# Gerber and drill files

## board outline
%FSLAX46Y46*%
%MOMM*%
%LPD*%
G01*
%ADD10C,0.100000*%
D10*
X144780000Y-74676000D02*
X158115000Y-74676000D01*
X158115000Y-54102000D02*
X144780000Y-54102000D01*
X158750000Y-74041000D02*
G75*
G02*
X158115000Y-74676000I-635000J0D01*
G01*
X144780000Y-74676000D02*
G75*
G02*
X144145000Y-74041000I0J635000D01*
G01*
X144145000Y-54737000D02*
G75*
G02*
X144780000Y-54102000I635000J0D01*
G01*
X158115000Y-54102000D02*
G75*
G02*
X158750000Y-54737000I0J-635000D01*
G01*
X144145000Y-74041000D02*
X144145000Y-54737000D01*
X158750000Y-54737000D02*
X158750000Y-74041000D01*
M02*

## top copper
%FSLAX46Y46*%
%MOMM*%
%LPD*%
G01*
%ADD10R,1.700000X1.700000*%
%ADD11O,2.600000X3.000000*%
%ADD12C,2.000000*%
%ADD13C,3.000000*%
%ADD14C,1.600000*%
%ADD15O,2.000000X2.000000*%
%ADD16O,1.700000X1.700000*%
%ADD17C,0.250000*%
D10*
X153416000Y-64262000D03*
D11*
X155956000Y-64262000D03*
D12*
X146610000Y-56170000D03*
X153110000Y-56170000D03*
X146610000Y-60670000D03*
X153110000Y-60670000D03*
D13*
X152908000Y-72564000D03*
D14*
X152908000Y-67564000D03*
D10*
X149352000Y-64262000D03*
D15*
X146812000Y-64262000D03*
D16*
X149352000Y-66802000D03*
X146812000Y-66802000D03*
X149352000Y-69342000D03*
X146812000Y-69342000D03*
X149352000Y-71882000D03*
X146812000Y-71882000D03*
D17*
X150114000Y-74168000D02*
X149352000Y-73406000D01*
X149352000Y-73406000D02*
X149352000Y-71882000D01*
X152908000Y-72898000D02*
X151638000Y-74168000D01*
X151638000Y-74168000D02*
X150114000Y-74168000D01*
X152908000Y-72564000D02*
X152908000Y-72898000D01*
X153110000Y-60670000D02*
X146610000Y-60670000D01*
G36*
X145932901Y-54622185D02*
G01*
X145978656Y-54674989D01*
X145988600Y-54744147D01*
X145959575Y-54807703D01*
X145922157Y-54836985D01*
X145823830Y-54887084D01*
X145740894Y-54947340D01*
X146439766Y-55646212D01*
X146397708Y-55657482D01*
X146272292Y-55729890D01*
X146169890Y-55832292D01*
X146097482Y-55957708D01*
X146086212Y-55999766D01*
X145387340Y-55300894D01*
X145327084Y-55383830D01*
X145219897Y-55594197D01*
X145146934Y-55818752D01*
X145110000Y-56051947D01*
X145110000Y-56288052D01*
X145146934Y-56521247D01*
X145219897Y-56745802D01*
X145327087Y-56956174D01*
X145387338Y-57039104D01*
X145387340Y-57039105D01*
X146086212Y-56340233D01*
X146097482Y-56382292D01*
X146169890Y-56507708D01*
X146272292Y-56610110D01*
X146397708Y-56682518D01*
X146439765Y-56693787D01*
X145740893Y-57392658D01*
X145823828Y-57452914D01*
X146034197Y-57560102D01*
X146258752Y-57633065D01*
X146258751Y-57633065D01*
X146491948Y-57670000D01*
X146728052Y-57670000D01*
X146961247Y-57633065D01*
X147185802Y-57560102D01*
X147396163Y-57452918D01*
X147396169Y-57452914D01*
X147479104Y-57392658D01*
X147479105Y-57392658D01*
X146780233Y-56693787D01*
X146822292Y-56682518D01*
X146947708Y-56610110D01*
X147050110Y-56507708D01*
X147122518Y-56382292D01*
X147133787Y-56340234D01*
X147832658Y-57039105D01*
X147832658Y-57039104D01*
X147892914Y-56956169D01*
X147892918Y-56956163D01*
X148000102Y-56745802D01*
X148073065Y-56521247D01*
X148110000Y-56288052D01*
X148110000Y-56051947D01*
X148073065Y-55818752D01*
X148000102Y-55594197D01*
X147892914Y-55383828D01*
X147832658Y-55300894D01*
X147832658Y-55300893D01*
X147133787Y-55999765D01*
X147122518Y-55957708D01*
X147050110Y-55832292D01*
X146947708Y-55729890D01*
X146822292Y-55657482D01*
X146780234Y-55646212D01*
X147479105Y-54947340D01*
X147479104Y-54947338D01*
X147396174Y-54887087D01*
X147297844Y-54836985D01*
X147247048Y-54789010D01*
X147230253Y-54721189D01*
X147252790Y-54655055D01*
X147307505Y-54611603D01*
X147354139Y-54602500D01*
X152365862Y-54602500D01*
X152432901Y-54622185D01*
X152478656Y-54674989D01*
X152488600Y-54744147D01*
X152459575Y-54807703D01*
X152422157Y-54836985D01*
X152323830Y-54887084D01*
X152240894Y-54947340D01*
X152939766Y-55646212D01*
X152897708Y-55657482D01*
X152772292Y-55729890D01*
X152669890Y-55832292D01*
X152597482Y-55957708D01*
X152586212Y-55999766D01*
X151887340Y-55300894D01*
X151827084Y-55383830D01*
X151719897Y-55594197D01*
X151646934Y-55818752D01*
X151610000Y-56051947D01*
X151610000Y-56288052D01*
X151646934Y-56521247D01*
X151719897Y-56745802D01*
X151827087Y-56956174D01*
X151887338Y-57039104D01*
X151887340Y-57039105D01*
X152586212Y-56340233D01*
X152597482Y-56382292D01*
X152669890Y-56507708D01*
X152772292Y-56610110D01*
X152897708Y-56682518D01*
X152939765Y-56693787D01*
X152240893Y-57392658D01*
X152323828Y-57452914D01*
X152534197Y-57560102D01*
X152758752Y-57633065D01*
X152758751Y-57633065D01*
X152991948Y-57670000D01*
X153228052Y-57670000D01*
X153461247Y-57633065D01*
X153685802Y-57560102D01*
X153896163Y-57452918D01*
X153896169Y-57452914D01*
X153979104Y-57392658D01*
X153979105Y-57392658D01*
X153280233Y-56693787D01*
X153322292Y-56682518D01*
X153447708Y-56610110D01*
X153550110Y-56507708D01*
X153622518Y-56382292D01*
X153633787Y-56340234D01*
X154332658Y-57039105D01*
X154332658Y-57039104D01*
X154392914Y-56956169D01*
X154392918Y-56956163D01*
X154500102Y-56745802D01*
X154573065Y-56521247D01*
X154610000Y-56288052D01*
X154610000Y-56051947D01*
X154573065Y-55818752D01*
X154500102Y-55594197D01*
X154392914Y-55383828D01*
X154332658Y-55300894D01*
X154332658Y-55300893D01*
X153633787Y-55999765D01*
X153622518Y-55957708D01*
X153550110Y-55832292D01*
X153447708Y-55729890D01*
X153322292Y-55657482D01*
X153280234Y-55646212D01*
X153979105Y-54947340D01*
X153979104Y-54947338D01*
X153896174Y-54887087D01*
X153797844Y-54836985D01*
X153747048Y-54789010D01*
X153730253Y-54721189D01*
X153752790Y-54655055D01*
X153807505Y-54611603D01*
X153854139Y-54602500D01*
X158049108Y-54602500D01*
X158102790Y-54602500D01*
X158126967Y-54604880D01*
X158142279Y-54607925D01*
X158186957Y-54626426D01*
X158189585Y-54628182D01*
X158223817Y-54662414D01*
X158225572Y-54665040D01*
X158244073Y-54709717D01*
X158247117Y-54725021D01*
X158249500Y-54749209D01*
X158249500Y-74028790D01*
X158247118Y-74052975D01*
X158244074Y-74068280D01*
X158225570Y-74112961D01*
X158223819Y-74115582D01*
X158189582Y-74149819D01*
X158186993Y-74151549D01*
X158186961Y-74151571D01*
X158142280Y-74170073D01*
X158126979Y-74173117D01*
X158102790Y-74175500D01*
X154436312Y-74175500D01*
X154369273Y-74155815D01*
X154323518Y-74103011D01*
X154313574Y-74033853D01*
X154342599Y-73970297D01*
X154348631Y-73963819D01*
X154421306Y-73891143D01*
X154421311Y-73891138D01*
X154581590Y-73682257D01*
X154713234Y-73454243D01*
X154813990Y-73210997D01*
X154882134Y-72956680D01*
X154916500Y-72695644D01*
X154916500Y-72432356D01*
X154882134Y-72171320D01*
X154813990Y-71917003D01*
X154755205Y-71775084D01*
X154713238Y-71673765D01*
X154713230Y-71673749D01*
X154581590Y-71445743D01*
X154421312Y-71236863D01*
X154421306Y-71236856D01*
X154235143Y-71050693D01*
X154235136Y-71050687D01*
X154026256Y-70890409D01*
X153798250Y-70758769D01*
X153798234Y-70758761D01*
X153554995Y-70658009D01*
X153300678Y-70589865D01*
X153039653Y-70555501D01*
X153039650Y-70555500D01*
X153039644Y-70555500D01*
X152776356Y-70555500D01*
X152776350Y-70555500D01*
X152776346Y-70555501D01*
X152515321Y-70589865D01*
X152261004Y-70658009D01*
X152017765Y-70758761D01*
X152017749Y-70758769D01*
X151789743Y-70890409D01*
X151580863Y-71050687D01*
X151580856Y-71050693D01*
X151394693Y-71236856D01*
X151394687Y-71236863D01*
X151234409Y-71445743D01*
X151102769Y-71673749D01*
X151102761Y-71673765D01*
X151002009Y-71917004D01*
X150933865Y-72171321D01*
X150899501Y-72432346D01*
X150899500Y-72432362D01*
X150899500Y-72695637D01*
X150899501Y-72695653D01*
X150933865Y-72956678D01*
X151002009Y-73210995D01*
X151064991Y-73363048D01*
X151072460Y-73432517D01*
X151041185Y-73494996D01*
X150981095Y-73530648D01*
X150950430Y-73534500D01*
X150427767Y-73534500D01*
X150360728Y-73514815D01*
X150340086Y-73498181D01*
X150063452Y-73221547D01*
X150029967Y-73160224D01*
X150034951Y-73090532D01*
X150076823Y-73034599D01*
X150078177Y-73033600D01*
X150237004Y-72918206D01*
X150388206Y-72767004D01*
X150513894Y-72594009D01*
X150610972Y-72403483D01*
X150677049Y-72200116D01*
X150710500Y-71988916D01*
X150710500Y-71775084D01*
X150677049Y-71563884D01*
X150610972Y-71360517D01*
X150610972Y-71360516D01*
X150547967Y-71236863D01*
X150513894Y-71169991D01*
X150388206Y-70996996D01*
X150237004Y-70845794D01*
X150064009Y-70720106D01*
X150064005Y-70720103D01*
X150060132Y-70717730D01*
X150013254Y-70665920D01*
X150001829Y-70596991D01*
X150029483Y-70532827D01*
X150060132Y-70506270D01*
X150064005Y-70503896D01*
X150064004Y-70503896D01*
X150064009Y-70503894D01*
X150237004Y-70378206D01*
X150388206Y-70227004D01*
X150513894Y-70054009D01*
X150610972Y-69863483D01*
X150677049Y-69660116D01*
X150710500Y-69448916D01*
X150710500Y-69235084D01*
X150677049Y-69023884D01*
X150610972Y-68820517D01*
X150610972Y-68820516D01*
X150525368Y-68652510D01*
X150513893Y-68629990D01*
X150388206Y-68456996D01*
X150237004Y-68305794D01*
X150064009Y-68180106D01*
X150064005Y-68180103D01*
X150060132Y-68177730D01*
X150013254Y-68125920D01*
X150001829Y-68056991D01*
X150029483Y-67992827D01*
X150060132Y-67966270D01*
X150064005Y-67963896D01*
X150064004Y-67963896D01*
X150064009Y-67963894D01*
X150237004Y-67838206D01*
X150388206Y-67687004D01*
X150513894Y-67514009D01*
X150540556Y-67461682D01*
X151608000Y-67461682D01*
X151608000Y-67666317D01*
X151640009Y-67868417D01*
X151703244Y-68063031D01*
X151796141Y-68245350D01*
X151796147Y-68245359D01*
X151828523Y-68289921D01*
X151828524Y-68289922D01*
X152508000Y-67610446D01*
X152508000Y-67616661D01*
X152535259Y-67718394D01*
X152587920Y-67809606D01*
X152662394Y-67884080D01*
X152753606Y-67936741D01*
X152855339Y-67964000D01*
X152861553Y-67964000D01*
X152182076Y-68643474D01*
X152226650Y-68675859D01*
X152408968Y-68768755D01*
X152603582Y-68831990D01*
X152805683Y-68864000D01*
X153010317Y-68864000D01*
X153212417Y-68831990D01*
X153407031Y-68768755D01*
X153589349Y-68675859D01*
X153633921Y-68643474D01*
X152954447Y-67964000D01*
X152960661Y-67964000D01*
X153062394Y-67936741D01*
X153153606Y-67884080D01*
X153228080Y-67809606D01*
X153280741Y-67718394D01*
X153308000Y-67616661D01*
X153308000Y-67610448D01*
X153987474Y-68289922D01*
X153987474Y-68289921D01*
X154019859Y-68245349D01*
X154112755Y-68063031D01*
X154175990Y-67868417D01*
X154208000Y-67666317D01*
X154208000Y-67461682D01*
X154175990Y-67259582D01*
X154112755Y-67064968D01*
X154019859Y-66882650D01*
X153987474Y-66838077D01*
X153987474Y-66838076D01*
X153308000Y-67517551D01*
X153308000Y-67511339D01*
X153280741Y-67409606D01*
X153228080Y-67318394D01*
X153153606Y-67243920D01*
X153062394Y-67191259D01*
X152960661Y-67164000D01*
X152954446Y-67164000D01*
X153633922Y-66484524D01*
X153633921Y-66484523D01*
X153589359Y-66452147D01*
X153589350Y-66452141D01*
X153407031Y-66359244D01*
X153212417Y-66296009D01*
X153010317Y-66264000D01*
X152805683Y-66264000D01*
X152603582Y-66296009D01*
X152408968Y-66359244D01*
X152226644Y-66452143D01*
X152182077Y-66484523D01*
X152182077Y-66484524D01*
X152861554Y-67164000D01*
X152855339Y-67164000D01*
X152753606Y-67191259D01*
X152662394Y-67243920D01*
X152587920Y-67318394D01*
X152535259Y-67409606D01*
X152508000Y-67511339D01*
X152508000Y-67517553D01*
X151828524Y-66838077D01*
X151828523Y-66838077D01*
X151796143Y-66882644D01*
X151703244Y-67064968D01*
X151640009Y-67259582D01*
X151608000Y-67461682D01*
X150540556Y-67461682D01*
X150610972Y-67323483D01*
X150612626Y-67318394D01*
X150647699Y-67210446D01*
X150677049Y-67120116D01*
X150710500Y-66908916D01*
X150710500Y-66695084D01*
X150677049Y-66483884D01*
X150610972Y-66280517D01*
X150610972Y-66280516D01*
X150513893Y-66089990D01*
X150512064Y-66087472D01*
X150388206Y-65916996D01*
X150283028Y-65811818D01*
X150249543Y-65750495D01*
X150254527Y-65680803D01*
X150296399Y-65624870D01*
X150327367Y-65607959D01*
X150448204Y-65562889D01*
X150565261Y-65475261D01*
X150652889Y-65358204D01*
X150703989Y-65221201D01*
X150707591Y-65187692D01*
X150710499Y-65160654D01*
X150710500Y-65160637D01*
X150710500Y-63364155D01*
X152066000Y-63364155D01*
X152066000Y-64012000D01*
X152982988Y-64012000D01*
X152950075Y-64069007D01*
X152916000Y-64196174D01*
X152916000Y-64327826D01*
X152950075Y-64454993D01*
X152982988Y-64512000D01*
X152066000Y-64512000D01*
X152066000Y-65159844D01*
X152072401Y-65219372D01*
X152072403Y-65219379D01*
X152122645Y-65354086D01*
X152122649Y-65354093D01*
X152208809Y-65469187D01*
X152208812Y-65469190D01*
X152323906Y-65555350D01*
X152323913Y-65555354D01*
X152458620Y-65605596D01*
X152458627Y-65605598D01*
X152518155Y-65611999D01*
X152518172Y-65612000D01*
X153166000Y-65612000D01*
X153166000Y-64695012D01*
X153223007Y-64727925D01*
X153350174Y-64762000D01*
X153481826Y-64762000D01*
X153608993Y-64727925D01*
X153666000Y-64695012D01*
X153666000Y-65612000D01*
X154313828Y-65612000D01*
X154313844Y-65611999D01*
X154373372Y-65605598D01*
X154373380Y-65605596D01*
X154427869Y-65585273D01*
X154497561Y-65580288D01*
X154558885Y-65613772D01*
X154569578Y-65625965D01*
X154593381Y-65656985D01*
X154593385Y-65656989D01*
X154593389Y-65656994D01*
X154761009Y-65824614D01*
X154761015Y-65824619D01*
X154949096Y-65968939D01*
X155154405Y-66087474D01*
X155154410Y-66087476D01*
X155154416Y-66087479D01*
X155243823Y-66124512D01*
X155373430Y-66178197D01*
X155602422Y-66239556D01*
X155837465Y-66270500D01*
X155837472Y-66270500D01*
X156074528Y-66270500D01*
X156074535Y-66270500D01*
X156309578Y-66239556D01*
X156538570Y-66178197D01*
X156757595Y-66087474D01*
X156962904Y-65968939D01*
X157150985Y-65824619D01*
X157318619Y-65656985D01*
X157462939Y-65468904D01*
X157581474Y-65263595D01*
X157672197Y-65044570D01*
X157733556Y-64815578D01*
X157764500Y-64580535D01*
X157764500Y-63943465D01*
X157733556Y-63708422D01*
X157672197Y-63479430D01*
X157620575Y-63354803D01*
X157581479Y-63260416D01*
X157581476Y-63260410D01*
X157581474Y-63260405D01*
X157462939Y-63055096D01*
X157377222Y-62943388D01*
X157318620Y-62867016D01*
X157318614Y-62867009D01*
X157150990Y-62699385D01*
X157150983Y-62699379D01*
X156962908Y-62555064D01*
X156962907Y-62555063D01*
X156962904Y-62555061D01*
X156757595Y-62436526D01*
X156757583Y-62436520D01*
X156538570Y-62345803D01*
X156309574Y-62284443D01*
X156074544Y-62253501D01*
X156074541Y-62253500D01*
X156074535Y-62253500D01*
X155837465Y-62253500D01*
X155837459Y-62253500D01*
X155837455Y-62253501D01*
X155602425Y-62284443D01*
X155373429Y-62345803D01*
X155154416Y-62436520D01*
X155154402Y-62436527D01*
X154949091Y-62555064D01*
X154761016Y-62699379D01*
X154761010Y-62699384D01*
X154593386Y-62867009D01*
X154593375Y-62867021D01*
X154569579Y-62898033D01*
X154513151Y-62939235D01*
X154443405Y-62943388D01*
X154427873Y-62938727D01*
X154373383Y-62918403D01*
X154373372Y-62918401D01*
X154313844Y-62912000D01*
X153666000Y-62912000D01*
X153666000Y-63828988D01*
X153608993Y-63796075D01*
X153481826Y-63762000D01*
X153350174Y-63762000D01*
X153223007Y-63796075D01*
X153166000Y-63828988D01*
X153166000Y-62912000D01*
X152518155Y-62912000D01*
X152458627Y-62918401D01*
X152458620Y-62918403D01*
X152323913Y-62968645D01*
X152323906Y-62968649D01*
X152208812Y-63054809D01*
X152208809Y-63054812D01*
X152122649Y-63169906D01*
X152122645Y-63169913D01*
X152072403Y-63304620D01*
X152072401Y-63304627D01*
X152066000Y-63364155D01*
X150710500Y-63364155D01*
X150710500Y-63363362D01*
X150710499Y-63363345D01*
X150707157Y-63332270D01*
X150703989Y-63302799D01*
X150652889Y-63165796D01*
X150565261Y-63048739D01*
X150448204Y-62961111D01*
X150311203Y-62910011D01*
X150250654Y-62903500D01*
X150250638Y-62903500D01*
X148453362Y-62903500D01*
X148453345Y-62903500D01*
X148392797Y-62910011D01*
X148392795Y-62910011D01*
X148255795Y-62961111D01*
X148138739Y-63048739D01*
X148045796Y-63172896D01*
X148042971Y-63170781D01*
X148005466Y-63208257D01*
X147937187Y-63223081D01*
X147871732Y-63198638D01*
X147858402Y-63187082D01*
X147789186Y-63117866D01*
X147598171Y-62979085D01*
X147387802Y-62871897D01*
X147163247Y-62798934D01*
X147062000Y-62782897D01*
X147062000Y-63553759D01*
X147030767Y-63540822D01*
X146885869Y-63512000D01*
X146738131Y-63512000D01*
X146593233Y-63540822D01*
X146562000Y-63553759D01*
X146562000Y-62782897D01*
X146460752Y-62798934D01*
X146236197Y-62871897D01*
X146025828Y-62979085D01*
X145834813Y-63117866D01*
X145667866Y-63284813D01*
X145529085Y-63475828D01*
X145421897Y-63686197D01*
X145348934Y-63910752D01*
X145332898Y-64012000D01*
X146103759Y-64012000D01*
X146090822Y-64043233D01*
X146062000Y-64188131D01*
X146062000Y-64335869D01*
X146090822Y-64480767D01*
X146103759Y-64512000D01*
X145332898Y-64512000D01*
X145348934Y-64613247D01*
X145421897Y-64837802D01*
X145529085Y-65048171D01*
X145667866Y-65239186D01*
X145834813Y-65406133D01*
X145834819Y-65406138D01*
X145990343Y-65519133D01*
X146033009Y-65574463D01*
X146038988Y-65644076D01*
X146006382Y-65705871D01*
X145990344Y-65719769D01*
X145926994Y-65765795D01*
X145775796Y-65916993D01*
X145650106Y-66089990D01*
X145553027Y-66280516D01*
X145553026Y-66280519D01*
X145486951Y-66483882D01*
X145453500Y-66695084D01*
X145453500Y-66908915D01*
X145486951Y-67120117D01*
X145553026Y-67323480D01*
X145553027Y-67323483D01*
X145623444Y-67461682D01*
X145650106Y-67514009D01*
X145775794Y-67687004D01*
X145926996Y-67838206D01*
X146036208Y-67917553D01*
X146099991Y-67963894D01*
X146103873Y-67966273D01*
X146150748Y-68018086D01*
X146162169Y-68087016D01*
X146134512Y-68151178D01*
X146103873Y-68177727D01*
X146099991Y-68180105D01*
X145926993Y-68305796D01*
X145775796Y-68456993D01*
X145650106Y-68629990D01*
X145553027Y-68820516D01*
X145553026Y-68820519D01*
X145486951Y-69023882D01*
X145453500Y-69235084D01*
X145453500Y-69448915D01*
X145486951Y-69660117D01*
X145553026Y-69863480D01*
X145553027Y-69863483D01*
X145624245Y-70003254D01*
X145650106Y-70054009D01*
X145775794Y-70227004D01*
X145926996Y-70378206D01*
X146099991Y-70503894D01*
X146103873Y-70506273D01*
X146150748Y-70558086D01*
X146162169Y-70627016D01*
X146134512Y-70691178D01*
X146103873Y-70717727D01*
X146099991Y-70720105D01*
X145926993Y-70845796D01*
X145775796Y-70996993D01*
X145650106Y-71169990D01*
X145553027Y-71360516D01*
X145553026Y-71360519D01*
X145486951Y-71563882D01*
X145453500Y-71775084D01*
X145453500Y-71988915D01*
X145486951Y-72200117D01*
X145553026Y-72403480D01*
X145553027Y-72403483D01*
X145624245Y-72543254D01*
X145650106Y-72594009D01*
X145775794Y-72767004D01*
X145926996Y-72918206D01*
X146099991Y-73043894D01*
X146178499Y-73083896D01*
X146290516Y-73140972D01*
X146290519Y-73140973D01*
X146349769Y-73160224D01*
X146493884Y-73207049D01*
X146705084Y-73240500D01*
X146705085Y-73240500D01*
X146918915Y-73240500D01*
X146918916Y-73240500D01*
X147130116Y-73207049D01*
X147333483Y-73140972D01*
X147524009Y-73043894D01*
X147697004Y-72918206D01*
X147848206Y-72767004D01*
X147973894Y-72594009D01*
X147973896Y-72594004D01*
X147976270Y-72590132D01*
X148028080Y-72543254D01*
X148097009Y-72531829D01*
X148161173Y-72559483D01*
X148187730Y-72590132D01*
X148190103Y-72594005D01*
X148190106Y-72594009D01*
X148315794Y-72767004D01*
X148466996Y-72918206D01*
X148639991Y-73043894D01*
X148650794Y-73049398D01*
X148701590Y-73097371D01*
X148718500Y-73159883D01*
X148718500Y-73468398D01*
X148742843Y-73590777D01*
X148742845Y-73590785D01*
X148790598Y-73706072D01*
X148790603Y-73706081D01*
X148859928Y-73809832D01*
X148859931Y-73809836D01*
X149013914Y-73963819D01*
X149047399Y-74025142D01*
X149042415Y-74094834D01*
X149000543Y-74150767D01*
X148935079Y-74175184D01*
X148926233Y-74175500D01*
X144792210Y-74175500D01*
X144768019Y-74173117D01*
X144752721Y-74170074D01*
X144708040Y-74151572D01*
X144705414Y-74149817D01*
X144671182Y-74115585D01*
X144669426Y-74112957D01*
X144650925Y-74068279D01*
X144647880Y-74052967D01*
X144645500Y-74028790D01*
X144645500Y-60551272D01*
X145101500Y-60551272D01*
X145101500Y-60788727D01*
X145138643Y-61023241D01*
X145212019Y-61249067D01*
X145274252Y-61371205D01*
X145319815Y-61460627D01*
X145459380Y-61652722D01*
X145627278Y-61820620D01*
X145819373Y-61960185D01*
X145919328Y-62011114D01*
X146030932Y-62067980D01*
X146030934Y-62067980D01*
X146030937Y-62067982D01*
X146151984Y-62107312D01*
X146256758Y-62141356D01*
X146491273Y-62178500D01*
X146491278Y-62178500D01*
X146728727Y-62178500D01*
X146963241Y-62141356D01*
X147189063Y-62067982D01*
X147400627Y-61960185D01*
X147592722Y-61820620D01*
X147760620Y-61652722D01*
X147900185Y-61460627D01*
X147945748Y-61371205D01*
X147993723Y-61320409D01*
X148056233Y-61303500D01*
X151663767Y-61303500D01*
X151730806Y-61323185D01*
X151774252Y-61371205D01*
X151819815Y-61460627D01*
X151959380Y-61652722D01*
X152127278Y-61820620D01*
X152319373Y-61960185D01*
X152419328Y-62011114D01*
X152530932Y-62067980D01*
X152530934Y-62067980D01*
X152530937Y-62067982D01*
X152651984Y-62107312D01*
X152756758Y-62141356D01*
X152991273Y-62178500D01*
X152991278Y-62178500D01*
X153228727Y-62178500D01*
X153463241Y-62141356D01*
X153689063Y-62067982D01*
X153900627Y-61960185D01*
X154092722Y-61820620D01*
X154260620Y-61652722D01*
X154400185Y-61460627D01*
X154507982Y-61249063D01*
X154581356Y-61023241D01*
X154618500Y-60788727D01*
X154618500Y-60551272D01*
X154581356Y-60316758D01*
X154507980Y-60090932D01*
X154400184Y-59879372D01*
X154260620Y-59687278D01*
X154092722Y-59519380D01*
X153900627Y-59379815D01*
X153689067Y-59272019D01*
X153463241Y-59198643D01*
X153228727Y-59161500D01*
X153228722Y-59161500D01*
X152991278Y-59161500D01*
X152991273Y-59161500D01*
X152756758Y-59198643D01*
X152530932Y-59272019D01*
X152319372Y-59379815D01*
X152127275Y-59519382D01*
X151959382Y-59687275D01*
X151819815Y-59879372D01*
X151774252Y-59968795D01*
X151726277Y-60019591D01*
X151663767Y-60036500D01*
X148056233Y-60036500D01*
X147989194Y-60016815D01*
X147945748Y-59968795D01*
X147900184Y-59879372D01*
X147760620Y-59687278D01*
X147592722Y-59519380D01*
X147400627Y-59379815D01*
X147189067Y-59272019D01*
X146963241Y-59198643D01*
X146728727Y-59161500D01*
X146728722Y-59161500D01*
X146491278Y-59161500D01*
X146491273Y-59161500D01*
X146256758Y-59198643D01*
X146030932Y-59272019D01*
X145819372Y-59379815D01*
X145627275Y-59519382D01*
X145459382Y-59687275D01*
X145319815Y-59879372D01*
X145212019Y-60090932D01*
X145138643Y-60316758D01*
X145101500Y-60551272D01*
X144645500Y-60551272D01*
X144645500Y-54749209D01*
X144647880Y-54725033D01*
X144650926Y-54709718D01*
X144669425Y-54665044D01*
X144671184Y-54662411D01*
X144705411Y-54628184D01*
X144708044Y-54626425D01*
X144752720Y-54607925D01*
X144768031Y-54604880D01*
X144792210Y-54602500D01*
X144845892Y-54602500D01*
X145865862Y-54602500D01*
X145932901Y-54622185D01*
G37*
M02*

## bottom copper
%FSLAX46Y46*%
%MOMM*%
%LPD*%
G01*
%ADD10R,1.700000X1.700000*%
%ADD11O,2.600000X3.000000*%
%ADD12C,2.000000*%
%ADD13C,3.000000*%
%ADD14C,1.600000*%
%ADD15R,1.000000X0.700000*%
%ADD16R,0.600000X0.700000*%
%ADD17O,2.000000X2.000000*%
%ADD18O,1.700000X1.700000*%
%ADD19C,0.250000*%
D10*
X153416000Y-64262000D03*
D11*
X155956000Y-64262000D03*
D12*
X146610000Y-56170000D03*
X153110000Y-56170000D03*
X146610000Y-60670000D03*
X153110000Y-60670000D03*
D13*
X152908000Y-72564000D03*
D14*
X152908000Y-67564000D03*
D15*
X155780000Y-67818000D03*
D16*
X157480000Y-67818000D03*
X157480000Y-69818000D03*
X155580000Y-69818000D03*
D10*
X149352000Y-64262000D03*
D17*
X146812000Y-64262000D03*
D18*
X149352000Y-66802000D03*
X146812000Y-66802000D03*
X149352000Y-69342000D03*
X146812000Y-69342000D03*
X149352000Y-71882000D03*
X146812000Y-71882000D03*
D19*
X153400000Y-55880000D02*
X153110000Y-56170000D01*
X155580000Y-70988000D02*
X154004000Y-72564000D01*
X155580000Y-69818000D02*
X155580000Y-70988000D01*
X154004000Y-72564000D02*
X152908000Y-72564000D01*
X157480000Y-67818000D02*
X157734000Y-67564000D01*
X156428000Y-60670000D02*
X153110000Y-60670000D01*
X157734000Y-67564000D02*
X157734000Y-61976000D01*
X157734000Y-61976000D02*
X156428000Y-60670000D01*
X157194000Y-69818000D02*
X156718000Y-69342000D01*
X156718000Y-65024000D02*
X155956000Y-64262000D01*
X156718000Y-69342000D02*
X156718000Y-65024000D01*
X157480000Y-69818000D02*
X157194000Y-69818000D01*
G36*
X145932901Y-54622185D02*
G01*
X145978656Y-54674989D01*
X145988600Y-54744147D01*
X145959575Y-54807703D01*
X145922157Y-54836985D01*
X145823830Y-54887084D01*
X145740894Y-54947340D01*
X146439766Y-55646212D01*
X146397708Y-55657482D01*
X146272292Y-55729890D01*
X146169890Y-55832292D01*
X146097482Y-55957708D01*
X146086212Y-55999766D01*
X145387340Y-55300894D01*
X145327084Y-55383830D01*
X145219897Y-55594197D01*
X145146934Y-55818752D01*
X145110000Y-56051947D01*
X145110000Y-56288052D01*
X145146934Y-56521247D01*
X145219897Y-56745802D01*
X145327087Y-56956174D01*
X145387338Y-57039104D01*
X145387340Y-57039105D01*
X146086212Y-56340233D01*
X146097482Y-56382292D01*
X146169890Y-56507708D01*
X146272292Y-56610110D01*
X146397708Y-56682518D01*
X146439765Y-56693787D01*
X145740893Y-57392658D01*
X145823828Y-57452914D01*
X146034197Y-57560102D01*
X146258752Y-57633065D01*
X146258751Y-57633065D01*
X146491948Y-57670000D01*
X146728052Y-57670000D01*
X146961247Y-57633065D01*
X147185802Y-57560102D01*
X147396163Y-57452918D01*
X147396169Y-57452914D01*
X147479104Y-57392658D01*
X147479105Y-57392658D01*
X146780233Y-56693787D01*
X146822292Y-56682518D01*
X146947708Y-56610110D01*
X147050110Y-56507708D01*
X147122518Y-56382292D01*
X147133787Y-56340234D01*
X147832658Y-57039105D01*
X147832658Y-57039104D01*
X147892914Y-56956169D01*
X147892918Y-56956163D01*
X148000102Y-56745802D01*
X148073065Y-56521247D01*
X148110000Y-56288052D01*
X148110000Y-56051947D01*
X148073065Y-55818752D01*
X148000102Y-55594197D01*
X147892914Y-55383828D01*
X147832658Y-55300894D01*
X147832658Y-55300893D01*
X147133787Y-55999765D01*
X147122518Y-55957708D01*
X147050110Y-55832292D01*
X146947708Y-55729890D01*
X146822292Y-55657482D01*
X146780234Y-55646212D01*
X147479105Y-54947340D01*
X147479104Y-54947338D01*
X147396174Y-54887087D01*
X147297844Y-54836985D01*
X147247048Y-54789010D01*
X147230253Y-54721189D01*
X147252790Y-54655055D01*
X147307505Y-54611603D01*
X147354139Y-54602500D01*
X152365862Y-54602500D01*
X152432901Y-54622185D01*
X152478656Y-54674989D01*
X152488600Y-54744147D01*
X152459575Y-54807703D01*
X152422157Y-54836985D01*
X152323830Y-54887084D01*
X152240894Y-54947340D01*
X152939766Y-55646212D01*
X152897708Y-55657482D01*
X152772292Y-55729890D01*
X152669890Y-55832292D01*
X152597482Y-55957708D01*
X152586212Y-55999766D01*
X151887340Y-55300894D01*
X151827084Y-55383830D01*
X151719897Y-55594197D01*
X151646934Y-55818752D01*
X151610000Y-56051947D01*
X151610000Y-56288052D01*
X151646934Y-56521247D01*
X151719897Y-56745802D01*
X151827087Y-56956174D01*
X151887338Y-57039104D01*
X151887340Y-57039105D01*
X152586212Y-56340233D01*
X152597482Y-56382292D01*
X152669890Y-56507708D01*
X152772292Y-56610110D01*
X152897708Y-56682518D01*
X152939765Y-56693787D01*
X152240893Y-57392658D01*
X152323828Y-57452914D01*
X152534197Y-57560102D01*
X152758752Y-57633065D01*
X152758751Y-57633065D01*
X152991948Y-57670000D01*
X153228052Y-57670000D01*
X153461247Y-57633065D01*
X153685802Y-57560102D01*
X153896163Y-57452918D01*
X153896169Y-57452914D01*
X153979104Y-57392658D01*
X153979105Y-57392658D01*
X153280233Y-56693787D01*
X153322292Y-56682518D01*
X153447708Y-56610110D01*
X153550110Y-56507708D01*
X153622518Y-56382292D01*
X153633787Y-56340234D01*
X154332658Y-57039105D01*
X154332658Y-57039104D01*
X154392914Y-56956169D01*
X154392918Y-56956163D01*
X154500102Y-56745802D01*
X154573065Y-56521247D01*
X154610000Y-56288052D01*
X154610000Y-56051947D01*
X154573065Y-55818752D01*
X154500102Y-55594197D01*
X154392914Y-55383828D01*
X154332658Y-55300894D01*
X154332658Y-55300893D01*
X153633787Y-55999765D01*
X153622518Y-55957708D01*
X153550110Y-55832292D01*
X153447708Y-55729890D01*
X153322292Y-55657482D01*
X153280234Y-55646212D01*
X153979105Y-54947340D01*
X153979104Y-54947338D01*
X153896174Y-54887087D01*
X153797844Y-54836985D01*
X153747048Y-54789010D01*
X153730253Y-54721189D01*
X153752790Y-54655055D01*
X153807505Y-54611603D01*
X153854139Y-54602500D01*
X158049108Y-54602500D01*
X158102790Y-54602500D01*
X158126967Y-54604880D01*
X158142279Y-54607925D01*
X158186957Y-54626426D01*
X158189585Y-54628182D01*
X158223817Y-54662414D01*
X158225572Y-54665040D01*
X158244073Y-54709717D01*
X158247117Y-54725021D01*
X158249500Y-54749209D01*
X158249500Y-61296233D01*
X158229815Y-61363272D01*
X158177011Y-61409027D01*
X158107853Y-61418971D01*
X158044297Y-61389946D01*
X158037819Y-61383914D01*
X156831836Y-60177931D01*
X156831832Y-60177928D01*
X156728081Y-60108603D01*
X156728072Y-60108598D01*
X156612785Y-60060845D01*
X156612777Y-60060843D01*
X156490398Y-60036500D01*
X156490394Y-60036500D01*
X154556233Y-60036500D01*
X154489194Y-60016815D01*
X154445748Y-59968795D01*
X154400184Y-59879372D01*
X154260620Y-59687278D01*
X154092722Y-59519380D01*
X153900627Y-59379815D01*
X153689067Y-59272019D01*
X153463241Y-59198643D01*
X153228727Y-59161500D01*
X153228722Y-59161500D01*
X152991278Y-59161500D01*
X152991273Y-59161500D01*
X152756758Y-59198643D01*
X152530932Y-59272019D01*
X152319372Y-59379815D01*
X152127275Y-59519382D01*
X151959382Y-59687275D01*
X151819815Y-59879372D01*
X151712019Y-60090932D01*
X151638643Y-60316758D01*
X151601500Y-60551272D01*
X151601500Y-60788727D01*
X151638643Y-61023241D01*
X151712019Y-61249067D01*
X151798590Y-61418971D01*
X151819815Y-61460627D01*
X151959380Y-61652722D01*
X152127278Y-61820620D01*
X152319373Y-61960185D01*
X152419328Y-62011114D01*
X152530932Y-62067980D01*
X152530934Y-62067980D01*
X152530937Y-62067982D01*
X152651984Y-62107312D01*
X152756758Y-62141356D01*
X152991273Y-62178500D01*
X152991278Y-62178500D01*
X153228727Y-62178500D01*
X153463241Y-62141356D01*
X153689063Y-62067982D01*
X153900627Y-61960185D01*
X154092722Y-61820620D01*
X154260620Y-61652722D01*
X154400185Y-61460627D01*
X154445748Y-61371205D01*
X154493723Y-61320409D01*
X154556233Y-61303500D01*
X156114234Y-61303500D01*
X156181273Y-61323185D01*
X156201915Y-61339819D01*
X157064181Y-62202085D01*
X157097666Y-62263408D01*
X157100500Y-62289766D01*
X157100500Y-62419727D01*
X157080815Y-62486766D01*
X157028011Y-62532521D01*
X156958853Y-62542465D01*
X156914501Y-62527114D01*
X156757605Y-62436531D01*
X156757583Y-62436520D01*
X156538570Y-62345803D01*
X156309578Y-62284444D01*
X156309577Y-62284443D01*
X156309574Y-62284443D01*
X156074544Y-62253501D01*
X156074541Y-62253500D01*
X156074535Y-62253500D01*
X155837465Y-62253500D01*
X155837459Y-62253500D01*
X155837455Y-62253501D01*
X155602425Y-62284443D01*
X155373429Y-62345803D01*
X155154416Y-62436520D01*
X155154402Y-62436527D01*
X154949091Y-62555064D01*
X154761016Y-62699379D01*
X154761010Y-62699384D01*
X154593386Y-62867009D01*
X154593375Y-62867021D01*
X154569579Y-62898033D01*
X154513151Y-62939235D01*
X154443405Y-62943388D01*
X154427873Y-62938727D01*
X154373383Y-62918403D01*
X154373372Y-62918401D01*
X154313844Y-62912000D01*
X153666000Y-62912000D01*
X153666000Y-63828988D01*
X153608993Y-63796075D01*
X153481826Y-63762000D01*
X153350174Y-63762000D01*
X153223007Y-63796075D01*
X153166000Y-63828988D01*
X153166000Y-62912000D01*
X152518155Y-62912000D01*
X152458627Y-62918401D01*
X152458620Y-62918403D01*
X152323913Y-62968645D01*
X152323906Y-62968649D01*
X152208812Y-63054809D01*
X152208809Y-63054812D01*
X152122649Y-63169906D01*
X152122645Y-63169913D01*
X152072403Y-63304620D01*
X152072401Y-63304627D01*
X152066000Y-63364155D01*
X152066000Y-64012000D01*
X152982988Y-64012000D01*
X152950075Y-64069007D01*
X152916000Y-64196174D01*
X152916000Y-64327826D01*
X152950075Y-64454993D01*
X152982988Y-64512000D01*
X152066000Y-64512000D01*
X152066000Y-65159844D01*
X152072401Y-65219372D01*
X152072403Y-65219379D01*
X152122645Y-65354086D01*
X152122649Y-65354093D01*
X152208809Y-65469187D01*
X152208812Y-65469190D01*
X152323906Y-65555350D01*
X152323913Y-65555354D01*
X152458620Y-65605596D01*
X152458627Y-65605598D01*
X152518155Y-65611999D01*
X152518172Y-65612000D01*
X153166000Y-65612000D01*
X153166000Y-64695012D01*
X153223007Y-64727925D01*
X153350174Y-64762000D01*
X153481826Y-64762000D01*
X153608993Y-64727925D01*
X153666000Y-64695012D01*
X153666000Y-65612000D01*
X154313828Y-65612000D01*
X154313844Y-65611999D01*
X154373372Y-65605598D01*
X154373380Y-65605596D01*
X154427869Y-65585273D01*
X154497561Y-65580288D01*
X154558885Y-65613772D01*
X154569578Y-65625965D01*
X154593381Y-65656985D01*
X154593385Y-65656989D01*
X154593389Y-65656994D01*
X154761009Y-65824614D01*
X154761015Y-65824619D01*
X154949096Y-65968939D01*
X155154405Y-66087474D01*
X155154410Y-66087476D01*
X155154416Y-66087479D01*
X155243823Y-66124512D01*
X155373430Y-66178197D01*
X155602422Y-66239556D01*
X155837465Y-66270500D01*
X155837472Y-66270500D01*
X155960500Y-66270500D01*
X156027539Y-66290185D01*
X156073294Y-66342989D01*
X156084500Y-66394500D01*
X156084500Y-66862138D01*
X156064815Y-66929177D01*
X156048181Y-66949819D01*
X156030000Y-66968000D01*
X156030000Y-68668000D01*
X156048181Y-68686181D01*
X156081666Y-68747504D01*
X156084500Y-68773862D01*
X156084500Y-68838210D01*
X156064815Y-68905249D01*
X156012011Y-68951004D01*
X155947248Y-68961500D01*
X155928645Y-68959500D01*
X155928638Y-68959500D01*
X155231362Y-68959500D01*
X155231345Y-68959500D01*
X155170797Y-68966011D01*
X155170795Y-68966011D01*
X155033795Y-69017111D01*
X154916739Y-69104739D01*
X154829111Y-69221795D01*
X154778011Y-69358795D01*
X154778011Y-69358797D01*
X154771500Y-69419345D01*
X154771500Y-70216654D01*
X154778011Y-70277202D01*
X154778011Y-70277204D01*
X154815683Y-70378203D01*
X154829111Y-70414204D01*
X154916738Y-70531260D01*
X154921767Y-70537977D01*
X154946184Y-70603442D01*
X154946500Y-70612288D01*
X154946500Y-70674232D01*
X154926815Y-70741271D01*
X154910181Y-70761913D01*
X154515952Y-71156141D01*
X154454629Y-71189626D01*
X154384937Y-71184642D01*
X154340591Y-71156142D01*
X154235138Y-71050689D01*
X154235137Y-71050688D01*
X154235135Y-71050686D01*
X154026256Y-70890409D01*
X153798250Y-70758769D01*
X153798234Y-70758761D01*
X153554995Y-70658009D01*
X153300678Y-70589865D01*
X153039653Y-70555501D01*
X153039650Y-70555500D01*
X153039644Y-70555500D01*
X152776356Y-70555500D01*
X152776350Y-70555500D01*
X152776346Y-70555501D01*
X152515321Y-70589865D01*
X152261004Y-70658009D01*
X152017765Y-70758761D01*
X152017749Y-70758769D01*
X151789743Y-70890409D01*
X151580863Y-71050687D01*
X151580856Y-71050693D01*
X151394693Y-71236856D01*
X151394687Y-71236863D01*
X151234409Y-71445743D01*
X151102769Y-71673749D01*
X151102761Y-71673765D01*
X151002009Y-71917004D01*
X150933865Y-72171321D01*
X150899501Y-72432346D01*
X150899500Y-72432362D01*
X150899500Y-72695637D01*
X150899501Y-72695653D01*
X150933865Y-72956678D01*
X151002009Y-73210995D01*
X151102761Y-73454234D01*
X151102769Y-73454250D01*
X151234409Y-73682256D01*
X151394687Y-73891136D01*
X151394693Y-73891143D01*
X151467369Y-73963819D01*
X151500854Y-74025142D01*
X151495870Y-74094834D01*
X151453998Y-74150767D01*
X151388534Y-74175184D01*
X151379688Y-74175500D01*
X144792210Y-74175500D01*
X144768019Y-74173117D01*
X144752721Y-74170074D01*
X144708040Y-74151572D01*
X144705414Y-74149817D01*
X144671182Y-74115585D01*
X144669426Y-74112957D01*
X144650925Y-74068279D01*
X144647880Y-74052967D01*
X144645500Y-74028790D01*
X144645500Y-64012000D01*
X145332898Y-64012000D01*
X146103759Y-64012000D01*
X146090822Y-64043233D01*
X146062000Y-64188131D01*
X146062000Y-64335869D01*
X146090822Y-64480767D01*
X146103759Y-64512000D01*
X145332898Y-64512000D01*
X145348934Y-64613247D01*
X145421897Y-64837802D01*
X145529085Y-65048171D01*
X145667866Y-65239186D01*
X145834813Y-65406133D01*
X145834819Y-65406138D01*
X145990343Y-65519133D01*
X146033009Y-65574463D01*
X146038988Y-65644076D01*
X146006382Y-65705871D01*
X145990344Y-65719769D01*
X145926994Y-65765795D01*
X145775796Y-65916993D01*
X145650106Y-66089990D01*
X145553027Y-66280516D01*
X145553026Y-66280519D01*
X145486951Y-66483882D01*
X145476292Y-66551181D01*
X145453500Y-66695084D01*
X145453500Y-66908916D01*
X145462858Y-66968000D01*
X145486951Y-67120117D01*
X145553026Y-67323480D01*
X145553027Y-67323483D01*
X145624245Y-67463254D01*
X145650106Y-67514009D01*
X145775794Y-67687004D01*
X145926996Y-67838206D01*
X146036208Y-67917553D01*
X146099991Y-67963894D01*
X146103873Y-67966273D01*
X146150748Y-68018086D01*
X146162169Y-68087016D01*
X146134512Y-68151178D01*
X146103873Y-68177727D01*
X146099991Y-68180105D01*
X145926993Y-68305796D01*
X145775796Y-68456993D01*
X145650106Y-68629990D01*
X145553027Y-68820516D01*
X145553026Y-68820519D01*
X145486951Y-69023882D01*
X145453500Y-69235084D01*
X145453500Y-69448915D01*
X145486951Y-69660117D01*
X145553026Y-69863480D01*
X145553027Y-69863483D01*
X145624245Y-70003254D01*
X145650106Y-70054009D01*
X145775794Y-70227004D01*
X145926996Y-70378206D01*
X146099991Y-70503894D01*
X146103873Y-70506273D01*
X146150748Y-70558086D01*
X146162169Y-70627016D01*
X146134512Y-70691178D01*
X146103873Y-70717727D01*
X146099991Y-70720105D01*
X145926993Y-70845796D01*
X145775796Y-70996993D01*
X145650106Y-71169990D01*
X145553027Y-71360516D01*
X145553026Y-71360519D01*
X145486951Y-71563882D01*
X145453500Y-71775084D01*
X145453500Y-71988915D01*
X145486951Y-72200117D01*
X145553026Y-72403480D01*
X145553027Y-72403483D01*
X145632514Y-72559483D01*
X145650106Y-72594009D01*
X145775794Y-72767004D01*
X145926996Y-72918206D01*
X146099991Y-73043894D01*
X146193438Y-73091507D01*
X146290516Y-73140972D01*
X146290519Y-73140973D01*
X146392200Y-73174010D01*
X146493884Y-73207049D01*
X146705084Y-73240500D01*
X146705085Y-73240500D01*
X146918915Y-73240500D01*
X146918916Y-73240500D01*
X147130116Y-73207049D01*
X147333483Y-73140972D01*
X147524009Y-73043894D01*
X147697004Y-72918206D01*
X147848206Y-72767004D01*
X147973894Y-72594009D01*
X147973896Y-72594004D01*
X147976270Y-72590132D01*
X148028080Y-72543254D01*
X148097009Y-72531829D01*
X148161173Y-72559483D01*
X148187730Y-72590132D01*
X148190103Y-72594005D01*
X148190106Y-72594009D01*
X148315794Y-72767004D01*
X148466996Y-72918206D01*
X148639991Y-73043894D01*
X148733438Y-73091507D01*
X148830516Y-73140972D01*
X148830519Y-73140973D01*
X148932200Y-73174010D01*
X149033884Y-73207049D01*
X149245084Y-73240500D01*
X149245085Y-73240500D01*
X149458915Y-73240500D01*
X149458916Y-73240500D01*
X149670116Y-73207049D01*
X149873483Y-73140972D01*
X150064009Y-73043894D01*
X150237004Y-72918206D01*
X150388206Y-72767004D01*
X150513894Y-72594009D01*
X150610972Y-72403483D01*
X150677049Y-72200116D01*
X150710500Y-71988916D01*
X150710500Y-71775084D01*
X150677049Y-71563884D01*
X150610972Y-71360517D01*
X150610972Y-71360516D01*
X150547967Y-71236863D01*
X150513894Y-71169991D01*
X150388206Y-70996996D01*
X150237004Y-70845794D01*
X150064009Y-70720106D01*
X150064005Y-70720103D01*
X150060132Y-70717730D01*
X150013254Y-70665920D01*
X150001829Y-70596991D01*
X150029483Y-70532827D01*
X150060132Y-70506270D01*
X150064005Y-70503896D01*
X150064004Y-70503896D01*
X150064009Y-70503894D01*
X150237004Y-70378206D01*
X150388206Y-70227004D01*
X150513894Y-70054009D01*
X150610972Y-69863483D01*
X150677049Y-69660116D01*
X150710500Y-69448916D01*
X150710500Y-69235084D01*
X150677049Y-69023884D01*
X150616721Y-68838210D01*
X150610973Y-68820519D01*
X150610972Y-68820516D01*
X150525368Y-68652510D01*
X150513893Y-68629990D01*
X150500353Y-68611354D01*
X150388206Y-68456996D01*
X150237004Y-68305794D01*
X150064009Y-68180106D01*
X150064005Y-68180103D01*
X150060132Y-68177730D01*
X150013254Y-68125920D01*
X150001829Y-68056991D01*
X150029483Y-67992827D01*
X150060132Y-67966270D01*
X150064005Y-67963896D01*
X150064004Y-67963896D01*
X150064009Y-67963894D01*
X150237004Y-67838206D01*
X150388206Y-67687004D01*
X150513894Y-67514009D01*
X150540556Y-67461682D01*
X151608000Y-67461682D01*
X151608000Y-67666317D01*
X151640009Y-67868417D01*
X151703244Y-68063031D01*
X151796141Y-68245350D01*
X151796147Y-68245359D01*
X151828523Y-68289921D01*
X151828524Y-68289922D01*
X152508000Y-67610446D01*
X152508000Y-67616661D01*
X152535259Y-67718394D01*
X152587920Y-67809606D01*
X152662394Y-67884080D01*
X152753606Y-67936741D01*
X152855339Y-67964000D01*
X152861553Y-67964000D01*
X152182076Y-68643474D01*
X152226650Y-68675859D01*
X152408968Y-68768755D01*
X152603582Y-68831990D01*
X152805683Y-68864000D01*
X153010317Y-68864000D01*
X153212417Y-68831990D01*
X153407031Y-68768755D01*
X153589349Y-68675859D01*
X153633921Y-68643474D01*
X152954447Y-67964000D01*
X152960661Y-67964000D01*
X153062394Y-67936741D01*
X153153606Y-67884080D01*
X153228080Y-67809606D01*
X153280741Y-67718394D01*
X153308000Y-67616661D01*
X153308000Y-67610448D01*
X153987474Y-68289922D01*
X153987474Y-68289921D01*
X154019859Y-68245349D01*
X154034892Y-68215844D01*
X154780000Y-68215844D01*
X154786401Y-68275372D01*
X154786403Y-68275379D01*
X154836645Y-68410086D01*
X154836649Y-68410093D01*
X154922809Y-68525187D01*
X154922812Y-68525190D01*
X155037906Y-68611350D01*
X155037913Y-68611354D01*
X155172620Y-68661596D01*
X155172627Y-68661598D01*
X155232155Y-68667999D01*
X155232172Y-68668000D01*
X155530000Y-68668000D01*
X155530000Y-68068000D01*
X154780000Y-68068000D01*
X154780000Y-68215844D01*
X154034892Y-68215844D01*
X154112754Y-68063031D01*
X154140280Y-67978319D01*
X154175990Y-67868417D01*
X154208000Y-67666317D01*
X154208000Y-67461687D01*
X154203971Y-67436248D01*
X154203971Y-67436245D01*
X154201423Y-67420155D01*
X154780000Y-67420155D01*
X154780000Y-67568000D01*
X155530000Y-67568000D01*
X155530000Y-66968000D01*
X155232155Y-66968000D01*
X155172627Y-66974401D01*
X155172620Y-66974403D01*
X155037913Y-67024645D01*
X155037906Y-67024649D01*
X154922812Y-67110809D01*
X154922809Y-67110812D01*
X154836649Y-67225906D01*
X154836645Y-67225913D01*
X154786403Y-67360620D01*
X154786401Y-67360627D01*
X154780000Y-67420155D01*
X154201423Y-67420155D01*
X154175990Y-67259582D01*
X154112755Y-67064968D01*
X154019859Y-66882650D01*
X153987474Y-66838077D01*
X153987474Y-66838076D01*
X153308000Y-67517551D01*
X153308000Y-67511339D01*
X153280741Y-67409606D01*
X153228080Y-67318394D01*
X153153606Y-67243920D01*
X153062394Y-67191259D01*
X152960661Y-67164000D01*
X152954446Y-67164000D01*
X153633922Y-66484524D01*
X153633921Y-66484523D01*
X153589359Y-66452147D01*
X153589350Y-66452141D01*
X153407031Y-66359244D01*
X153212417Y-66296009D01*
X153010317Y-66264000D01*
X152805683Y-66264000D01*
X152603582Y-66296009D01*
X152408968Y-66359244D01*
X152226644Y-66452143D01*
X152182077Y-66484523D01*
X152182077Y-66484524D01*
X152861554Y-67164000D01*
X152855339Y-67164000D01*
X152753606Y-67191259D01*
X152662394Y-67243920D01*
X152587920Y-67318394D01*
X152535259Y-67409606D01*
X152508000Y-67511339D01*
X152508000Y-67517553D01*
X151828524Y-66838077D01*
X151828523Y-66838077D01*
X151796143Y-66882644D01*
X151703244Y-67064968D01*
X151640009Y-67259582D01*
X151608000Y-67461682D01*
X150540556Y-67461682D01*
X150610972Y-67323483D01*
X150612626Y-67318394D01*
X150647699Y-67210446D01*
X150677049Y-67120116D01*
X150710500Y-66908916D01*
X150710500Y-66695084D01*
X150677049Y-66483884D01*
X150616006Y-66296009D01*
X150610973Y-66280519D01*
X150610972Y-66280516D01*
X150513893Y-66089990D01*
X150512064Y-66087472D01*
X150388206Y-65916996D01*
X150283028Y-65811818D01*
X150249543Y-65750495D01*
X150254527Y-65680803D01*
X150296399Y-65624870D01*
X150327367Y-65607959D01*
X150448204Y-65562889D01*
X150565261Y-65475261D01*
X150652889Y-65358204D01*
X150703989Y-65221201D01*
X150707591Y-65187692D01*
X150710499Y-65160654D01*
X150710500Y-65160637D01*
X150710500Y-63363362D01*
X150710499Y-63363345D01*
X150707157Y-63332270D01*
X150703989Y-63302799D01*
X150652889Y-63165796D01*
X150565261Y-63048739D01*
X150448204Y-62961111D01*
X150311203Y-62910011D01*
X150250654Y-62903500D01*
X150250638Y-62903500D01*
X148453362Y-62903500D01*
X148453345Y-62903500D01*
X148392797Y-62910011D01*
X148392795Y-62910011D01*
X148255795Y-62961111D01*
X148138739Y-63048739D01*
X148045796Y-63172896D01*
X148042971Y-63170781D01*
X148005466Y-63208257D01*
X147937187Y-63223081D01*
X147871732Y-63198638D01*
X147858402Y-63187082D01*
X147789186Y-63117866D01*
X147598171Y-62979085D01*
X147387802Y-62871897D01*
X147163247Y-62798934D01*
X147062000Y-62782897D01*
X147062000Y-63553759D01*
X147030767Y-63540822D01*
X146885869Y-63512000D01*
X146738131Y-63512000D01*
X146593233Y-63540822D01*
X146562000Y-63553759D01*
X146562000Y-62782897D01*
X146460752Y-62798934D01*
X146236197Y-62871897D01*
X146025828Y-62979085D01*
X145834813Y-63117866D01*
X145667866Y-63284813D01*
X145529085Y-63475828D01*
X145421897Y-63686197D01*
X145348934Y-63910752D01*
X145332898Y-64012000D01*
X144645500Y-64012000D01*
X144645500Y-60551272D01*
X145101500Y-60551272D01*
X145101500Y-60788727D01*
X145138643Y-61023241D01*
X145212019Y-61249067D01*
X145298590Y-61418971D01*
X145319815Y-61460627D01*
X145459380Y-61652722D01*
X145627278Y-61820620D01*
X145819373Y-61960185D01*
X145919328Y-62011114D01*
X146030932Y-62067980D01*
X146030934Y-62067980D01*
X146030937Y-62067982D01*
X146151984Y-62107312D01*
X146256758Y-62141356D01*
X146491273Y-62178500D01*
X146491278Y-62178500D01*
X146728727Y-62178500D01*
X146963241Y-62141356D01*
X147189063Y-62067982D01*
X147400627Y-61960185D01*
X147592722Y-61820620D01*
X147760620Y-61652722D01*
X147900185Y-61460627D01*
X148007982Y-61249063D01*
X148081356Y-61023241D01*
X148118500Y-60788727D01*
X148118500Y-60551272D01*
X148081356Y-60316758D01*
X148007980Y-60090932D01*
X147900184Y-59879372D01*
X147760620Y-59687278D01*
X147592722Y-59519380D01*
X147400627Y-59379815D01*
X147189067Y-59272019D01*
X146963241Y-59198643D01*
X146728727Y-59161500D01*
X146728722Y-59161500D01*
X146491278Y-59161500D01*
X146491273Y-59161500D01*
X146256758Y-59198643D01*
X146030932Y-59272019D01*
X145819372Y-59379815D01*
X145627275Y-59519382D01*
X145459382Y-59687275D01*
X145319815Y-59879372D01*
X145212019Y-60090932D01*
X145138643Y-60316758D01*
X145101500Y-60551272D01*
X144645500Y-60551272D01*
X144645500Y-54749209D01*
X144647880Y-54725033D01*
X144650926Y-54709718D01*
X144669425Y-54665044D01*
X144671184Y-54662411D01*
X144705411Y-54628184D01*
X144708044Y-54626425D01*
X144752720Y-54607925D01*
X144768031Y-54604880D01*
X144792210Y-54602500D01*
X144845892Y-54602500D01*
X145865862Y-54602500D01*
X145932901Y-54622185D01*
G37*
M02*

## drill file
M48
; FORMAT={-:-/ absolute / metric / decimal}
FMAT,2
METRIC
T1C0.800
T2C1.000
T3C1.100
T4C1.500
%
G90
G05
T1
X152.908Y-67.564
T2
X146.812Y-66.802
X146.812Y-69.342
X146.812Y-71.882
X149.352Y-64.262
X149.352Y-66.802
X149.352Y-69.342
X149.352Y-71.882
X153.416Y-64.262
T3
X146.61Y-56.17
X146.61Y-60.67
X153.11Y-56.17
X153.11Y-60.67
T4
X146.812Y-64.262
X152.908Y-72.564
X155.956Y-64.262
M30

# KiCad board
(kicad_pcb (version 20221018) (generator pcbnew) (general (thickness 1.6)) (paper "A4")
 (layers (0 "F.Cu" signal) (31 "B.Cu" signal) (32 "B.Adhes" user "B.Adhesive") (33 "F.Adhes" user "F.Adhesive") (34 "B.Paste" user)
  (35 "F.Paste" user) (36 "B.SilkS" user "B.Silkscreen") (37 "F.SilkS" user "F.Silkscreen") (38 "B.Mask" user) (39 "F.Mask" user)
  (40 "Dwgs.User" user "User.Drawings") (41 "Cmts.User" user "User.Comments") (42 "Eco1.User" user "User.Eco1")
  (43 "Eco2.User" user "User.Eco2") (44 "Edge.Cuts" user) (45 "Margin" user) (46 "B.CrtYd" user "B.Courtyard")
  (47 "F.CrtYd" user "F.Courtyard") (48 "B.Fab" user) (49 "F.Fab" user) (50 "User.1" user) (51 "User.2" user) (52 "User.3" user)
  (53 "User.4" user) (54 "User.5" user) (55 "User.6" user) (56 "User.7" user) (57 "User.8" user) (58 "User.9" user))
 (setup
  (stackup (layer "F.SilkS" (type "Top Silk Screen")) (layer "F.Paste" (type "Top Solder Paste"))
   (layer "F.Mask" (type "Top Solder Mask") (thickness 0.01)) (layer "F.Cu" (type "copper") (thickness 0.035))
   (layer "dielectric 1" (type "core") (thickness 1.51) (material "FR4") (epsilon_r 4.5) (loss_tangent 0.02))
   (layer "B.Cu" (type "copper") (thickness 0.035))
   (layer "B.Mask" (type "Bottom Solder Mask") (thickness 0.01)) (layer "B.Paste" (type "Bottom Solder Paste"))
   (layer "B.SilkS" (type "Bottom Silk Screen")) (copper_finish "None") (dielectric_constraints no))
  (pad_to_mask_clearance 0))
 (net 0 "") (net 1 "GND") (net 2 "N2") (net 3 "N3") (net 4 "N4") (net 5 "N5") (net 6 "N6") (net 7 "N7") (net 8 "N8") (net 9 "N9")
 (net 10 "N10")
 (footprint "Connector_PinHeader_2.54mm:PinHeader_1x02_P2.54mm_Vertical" (layer "F.Cu") (at 153.416 64.262 90)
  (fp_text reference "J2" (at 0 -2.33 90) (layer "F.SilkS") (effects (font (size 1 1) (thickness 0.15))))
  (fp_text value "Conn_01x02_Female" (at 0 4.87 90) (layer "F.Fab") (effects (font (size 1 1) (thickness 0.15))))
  (pad "1" thru_hole rect (at 0 0 90) (size 1.7 1.7) (drill 1) (layers "*.Cu" "*.Mask") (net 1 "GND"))
  (pad "2" thru_hole oval (at 0 2.54 90) (size 3 2.6) (drill 1.5) (layers "*.Cu" "*.Mask") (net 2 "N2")))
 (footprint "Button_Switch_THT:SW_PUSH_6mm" (layer "F.Cu") (at 146.61 56.17)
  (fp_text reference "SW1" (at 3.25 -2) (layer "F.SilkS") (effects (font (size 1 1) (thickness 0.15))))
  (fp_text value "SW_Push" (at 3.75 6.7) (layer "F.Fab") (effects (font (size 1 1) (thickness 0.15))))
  (pad "1" thru_hole circle (at 0 0 90) (size 2 2) (drill 1.1) (layers "*.Cu" "*.Mask") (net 1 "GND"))
  (pad "1" thru_hole circle (at 6.5 0 90) (size 2 2) (drill 1.1) (layers "*.Cu" "*.Mask") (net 1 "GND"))
  (pad "2" thru_hole circle (at 0 4.5 90) (size 2 2) (drill 1.1) (layers "*.Cu" "*.Mask") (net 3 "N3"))
  (pad "2" thru_hole circle (at 6.5 4.5 90) (size 2 2) (drill 1.1) (layers "*.Cu" "*.Mask") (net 3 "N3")))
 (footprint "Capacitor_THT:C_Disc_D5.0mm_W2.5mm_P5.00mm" (layer "F.Cu") (at 152.908 72.564 90)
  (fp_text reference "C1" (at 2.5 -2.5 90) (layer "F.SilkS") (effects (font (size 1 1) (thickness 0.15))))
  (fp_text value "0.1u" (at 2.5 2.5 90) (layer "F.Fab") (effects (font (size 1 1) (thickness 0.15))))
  (pad "1" thru_hole circle (at 0 0 90) (size 3 3) (drill 1.5) (layers "*.Cu" "*.Mask") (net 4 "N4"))
  (pad "2" thru_hole circle (at 5 0 90) (size 1.6 1.6) (drill 0.8) (layers "*.Cu" "*.Mask") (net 1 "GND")))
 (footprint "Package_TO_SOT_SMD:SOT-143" (layer "B.Cu") (at 156.53 68.818 -90)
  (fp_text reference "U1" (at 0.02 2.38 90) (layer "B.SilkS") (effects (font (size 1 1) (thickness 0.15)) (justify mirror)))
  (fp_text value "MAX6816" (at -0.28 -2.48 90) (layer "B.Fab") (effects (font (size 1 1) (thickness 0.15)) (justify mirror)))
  (pad "1" smd rect (at -1 0.75 270) (size 0.7 1) (layers "B.Cu" "B.Paste" "B.Mask") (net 1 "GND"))
  (pad "2" smd rect (at -1 -0.95 270) (size 0.7 0.6) (layers "B.Cu" "B.Paste" "B.Mask") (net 3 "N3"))
  (pad "3" smd rect (at 1 -0.95 270) (size 0.7 0.6) (layers "B.Cu" "B.Paste" "B.Mask") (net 2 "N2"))
  (pad "4" smd rect (at 1 0.95 270) (size 0.7 0.6) (layers "B.Cu" "B.Paste" "B.Mask") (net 4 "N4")))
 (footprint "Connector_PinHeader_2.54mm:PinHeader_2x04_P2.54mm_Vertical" (layer "B.Cu") (at 149.352 64.262 180)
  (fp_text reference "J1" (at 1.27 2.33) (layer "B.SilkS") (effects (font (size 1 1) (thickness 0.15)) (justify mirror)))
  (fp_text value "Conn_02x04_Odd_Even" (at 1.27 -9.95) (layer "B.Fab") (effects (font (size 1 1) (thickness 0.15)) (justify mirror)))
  (pad "1" thru_hole rect (at 0 0 180) (size 1.7 1.7) (drill 1) (layers "*.Cu" "*.Mask") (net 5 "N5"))
  (pad "2" thru_hole oval (at 2.54 0 180) (size 2 2) (drill 1.5) (layers "*.Cu" "*.Mask") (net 1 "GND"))
  (pad "3" thru_hole oval (at 0 -2.54 180) (size 1.7 1.7) (drill 1) (layers "*.Cu" "*.Mask") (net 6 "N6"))
  (pad "4" thru_hole oval (at 2.54 -2.54 180) (size 1.7 1.7) (drill 1) (layers "*.Cu" "*.Mask") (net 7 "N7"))
  (pad "5" thru_hole oval (at 0 -5.08 180) (size 1.7 1.7) (drill 1) (layers "*.Cu" "*.Mask") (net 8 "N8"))
  (pad "6" thru_hole oval (at 2.54 -5.08 180) (size 1.7 1.7) (drill 1) (layers "*.Cu" "*.Mask") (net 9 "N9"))
  (pad "7" thru_hole oval (at 0 -7.62 180) (size 1.7 1.7) (drill 1) (layers "*.Cu" "*.Mask") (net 4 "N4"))
  (pad "8" thru_hole oval (at 2.54 -7.62 180) (size 1.7 1.7) (drill 1) (layers "*.Cu" "*.Mask") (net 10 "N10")))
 (gr_line (start 144.78 74.676) (end 158.115 74.676) (stroke (width 0.1) (type default)) (layer "Edge.Cuts"))
 (gr_line (start 158.115 54.102) (end 144.78 54.102) (stroke (width 0.1) (type default)) (layer "Edge.Cuts"))
 (gr_arc (start 158.75 74.041) (mid 158.564013 74.490013) (end 158.115 74.676) (stroke (width 0.1) (type default)) (layer "Edge.Cuts"))
 (gr_arc (start 144.78 74.676) (mid 144.330987 74.490013) (end 144.145 74.041) (stroke (width 0.1) (type default)) (layer "Edge.Cuts"))
 (gr_arc (start 144.145 54.737) (mid 144.330987 54.287987) (end 144.78 54.102) (stroke (width 0.1) (type default)) (layer "Edge.Cuts"))
 (gr_arc (start 158.115 54.102) (mid 158.564013 54.287987) (end 158.75 54.737) (stroke (width 0.1) (type default)) (layer "Edge.Cuts"))
 (gr_line (start 144.145 74.041) (end 144.145 54.737) (stroke (width 0.1) (type default)) (layer "Edge.Cuts"))
 (gr_line (start 158.75 54.737) (end 158.75 74.041) (stroke (width 0.1) (type default)) (layer "Edge.Cuts"))
 (segment (start 153.4 55.88) (end 153.11 56.17) (width 0.25) (layer "B.Cu") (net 1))
 (segment (start 150.114 74.168) (end 149.352 73.406) (width 0.25) (layer "F.Cu") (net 4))
 (segment (start 149.352 73.406) (end 149.352 71.882) (width 0.25) (layer "F.Cu") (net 4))
 (segment (start 152.908 72.898) (end 151.638 74.168) (width 0.25) (layer "F.Cu") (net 4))
 (segment (start 151.638 74.168) (end 150.114 74.168) (width 0.25) (layer "F.Cu") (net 4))
 (segment (start 152.908 72.564) (end 152.908 72.898) (width 0.25) (layer "F.Cu") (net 4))
 (segment (start 155.58 70.988) (end 154.004 72.564) (width 0.25) (layer "B.Cu") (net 4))
 (segment (start 155.58 69.818) (end 155.58 70.988) (width 0.25) (layer "B.Cu") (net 4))
 (segment (start 154.004 72.564) (end 152.908 72.564) (width 0.25) (layer "B.Cu") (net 4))
 (segment (start 153.11 60.67) (end 146.61 60.67) (width 0.25) (layer "F.Cu") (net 3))
 (segment (start 157.48 67.818) (end 157.734 67.564) (width 0.25) (layer "B.Cu") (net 3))
 (segment (start 156.428 60.67) (end 153.11 60.67) (width 0.25) (layer "B.Cu") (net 3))
 (segment (start 157.734 67.564) (end 157.734 61.976) (width 0.25) (layer "B.Cu") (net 3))
 (segment (start 157.734 61.976) (end 156.428 60.67) (width 0.25) (layer "B.Cu") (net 3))
 (segment (start 157.194 69.818) (end 156.718 69.342) (width 0.25) (layer "B.Cu") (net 2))
 (segment (start 156.718 65.024) (end 155.956 64.262) (width 0.25) (layer "B.Cu") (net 2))
 (segment (start 156.718 69.342) (end 156.718 65.024) (width 0.25) (layer "B.Cu") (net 2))
 (segment (start 157.48 69.818) (end 157.194 69.818) (width 0.25) (layer "B.Cu") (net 2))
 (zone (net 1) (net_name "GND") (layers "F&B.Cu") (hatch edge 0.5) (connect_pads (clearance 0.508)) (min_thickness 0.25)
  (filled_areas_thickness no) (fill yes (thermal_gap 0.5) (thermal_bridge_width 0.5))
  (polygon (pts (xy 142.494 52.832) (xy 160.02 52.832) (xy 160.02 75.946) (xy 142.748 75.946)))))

